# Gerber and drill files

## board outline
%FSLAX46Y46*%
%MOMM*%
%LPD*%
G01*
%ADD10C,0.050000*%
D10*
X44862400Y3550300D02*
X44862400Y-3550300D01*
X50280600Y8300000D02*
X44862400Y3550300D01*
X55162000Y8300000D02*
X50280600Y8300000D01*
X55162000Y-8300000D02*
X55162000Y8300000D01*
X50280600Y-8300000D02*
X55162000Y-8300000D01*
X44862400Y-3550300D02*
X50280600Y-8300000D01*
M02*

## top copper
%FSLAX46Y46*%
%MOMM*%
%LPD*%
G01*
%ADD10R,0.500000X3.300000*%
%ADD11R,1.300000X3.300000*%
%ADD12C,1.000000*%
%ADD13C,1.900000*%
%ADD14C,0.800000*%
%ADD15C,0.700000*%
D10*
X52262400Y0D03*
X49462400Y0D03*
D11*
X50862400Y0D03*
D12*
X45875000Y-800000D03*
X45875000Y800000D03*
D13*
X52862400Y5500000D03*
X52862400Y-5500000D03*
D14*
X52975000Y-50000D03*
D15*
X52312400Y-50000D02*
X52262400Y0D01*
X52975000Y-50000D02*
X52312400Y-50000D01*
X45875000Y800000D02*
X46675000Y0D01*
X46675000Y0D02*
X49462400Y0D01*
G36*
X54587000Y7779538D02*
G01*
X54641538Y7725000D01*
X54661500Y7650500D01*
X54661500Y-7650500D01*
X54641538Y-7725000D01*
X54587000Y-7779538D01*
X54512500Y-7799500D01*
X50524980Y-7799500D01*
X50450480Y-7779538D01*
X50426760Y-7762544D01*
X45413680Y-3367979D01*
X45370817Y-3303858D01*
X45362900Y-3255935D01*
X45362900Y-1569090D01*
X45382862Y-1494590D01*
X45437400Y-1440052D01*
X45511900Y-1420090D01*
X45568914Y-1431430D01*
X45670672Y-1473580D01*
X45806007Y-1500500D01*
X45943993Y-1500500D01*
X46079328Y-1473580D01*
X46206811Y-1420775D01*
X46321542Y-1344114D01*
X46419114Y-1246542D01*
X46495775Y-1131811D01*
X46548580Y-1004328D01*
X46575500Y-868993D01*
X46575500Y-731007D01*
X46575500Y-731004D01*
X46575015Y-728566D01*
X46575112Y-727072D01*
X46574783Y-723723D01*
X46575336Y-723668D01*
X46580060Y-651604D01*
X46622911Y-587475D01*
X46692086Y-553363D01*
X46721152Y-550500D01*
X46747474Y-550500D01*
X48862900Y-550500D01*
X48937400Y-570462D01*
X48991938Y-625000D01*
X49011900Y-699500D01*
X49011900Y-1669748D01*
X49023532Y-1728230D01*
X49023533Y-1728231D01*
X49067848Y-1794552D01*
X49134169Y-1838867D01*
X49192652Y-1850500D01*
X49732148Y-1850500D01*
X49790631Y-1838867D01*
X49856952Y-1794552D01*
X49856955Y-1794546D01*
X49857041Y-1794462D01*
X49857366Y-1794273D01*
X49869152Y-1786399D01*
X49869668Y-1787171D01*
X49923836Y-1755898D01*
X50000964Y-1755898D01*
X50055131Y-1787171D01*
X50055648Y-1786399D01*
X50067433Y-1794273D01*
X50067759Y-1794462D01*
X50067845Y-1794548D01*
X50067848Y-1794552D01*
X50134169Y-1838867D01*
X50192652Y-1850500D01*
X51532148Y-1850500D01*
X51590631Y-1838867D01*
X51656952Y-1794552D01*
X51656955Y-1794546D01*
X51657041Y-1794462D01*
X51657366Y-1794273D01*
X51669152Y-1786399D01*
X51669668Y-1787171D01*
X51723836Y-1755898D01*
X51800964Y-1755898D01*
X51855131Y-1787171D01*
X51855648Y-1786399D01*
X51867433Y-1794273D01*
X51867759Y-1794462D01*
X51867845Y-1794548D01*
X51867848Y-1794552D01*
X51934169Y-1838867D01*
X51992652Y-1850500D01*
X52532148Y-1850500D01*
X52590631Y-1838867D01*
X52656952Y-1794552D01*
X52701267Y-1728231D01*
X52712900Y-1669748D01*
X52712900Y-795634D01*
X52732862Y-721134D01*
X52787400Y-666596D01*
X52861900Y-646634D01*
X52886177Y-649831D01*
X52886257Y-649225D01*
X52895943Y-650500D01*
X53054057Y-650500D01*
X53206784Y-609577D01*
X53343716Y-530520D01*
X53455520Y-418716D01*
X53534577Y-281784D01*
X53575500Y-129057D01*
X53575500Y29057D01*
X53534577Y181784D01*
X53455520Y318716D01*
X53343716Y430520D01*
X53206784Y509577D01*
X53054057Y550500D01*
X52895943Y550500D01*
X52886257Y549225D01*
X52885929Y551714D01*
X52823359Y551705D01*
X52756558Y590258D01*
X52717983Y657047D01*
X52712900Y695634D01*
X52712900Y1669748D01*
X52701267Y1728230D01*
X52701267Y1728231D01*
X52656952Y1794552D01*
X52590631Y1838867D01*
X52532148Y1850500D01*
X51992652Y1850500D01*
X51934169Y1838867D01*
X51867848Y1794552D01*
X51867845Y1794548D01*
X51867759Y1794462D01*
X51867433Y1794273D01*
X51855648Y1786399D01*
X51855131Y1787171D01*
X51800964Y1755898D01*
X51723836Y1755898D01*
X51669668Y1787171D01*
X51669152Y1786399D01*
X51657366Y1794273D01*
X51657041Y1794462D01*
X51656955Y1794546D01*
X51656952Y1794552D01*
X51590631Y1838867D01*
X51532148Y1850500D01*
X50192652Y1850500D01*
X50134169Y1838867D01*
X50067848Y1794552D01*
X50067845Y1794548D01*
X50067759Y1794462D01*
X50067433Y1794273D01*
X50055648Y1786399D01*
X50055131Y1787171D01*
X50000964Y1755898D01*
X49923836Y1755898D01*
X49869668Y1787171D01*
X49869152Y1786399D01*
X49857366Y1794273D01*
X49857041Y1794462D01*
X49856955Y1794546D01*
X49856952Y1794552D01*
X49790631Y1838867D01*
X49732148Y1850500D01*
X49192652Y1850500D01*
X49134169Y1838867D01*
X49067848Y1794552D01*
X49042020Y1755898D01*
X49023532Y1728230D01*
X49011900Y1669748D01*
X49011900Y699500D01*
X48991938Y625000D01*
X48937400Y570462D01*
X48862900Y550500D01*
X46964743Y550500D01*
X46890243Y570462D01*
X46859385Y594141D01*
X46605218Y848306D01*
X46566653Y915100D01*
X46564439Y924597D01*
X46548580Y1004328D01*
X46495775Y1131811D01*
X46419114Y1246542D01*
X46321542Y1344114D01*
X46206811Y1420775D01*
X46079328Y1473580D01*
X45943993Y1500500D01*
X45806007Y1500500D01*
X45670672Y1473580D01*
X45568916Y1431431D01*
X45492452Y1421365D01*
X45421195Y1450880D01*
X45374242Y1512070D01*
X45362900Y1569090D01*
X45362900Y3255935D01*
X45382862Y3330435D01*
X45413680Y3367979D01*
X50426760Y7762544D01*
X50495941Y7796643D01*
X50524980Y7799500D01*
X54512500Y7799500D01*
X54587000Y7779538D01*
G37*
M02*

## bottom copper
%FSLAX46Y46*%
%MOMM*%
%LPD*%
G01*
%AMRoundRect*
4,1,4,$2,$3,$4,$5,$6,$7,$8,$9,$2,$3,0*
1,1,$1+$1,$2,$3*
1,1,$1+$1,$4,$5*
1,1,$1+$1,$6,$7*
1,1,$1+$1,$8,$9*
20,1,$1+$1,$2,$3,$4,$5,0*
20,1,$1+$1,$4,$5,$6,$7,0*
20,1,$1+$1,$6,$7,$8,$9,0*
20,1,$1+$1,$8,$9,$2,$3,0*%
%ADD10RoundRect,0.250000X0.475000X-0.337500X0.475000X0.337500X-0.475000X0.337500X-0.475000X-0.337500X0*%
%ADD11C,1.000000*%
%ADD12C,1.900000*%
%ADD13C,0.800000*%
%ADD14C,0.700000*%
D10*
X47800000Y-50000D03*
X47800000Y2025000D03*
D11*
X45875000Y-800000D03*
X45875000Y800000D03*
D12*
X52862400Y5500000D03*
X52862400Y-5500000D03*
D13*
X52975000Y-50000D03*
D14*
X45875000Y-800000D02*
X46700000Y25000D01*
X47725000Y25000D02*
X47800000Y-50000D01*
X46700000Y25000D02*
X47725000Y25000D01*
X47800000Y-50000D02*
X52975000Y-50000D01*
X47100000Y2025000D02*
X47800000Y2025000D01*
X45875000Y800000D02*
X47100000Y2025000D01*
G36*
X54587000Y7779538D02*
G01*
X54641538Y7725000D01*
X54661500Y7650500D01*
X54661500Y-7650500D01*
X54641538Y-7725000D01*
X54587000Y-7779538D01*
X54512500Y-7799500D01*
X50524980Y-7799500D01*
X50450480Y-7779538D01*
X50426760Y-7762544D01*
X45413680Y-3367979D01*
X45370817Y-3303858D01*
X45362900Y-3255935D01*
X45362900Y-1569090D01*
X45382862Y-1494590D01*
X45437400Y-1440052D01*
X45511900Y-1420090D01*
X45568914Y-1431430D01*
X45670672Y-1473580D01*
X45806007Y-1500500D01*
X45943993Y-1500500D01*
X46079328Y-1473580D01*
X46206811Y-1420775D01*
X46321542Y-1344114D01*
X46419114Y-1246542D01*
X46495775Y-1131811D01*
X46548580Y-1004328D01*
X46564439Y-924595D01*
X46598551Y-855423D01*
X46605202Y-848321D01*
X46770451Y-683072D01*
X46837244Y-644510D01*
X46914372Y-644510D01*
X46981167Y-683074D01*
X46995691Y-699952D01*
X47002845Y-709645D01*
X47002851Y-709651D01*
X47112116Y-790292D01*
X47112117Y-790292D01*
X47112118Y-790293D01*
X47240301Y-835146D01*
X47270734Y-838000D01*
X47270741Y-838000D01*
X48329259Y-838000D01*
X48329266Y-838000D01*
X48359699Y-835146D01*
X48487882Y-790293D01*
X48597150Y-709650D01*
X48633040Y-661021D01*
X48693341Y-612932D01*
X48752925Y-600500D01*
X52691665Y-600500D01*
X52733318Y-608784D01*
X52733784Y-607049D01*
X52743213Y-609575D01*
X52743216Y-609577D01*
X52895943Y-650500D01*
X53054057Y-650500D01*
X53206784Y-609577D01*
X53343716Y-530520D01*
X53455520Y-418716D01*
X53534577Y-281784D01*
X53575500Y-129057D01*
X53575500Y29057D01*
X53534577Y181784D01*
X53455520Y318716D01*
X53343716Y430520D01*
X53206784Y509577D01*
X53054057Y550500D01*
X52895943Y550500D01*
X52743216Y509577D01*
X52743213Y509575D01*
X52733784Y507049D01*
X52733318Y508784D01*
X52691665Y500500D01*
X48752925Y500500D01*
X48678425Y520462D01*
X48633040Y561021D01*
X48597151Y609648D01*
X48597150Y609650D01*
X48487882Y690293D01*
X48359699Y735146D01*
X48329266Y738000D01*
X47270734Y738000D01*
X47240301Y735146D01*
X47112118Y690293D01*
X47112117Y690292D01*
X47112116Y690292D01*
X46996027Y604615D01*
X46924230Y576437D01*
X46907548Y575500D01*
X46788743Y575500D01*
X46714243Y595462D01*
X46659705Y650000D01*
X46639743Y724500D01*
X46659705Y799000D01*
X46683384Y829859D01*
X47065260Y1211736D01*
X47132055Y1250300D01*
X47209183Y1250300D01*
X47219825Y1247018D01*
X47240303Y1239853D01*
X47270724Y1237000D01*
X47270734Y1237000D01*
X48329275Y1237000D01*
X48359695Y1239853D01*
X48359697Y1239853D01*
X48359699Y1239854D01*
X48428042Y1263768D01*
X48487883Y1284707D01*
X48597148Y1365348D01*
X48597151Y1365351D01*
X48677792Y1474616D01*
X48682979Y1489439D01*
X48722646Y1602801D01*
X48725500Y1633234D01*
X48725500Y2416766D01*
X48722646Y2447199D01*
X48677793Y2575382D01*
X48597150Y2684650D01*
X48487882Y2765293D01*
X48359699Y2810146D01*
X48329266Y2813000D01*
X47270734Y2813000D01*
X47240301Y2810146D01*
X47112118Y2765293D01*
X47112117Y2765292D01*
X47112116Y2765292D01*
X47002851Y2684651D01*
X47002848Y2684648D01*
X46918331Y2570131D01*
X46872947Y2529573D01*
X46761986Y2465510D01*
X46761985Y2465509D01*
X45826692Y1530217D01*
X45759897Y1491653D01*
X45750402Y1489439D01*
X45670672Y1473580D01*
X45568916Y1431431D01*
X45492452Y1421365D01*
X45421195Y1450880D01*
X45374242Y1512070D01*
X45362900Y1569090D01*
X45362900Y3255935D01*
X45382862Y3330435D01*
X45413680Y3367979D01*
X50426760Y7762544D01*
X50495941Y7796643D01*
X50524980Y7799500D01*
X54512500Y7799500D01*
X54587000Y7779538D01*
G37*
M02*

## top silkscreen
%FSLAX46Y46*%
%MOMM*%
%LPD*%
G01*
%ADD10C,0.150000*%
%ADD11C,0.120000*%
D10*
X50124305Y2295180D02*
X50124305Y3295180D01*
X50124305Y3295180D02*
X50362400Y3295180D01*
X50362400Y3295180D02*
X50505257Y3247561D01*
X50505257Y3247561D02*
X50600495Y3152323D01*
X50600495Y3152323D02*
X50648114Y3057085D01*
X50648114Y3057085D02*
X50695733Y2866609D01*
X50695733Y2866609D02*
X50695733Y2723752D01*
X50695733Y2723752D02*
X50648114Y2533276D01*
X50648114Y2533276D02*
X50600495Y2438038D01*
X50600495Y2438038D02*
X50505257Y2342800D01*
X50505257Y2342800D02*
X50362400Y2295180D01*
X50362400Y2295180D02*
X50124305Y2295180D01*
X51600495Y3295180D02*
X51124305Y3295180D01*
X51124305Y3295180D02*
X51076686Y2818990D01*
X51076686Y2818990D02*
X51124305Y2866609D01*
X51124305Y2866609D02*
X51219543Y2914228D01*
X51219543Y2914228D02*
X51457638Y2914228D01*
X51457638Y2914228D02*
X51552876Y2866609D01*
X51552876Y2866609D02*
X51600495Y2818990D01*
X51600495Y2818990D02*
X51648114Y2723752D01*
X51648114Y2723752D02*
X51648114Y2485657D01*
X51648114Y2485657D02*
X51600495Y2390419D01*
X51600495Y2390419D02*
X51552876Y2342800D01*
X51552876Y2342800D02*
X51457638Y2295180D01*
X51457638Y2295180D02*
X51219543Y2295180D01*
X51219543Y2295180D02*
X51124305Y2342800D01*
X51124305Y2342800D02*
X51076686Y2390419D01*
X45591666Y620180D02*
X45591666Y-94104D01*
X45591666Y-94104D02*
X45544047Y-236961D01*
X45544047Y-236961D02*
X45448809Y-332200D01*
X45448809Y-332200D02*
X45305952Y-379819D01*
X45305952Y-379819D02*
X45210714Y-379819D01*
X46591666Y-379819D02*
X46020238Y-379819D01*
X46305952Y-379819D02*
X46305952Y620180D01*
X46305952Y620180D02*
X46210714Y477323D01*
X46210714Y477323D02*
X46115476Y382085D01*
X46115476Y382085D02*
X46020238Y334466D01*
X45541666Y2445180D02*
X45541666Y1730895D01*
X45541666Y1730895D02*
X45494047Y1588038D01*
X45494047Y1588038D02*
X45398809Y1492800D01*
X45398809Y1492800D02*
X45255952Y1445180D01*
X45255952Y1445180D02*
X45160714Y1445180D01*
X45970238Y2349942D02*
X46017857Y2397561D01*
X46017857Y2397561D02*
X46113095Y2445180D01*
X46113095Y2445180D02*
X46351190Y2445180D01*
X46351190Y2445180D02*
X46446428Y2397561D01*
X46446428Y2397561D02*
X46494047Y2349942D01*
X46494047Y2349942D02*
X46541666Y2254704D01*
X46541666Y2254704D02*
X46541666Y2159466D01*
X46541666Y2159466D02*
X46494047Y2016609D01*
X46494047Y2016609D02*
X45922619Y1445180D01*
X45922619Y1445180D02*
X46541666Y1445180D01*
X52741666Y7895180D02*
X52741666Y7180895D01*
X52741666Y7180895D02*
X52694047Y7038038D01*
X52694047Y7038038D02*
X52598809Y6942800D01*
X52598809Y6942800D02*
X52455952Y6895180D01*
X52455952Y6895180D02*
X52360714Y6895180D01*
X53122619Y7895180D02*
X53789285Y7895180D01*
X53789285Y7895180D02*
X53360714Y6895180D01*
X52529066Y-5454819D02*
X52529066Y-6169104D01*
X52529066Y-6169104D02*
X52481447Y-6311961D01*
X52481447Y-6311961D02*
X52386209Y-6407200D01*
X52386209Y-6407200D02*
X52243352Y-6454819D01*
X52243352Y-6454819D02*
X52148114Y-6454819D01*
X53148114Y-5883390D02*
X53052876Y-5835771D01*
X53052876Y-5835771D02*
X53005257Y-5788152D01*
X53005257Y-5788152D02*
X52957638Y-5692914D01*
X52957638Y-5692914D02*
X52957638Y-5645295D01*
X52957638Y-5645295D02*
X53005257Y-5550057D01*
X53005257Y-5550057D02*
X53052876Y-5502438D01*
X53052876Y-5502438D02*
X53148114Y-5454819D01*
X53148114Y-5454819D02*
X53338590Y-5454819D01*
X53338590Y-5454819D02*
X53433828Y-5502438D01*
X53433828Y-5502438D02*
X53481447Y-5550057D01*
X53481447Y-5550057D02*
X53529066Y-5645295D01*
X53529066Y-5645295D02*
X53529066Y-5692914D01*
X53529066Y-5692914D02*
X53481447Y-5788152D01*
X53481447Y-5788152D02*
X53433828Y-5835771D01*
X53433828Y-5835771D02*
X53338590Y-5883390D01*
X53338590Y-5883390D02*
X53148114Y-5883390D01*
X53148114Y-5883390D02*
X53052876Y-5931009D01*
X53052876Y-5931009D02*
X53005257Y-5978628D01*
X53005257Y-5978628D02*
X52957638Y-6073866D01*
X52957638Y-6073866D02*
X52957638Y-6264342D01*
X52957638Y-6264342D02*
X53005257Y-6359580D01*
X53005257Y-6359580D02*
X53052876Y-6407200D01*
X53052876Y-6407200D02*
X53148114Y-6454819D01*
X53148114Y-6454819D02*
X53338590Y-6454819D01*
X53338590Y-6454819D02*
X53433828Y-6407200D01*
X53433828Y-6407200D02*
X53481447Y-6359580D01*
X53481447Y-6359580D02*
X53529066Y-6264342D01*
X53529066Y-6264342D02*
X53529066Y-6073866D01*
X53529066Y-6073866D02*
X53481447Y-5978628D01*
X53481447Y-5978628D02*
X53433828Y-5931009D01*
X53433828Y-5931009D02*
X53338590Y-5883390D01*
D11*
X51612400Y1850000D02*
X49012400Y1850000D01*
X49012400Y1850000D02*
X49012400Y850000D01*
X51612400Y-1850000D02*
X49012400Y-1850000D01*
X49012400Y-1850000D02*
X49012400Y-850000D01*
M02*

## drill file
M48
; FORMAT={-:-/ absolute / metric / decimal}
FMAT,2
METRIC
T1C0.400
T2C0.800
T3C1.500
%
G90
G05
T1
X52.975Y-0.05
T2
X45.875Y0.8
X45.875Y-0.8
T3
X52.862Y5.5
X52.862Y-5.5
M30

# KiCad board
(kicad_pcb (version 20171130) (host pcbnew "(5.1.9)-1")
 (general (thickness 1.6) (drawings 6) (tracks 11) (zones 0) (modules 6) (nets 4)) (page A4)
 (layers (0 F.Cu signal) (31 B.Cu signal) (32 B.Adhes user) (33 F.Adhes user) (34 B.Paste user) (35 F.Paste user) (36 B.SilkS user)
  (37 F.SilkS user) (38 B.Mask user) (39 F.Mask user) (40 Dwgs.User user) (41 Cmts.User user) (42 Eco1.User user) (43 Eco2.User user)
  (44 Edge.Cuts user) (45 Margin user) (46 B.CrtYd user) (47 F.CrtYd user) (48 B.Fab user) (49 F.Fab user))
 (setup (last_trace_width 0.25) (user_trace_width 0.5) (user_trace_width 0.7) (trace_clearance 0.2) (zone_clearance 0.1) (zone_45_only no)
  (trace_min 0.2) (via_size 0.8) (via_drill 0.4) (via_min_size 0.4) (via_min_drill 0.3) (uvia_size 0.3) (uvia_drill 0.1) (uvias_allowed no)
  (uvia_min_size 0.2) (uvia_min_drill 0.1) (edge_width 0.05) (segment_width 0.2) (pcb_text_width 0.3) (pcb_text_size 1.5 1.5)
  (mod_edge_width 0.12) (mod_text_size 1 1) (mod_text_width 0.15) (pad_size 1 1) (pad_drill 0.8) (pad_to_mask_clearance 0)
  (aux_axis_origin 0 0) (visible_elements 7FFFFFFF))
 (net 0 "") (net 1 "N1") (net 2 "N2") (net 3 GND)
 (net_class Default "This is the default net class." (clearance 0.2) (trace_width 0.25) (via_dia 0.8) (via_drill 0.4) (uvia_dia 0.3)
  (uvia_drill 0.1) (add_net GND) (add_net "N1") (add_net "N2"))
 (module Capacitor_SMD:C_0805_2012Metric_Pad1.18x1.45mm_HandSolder (layer B.Cu) (at 47.8 -0.9875 90)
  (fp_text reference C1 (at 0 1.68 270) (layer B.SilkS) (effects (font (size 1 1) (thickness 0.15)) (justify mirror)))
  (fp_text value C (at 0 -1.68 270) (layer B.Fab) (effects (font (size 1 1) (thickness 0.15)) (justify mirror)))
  (pad 1 smd roundrect (at -1.0375 0 90) (size 1.175 1.45) (layers B.Cu B.Paste B.Mask) (roundrect_rratio 0.2127659574468085) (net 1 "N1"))
  (pad 2 smd roundrect (at 1.0375 0 90) (size 1.175 1.45) (layers B.Cu B.Paste B.Mask) (roundrect_rratio 0.2127659574468085) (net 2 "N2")))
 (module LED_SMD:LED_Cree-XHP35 (layer F.Cu) (at 50.8624 0)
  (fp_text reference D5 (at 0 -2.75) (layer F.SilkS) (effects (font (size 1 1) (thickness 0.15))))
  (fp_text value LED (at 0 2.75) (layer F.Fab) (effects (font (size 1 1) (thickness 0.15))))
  (fp_line (start 0.75 -1.85) (end -1.85 -1.85) (layer F.SilkS) (width 0.12))
  (fp_line (start -1.85 -1.85) (end -1.85 -0.85) (layer F.SilkS) (width 0.12))
  (fp_line (start 0.75 1.85) (end -1.85 1.85) (layer F.SilkS) (width 0.12))
  (fp_line (start -1.85 1.85) (end -1.85 0.85) (layer F.SilkS) (width 0.12))
  (pad 2 smd rect (at 1.4 0) (size 0.5 3.3) (layers F.Cu F.Paste F.Mask) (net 1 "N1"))
  (pad 1 smd rect (at -1.4 0) (size 0.5 3.3) (layers F.Cu F.Paste F.Mask) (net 2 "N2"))
  (pad 3 smd rect (at 0 0) (size 1.3 3.3) (layers F.Cu F.Mask)) (pad "" smd rect (at 0 1) (size 1.01 0.75) (layers F.Paste))
  (pad "" smd rect (at 0 -1) (size 1.01 0.75) (layers F.Paste)) (pad "" smd rect (at 0 0) (size 1.01 0.75) (layers F.Paste)))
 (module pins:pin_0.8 (layer F.Cu) (at 45.925 -0.575)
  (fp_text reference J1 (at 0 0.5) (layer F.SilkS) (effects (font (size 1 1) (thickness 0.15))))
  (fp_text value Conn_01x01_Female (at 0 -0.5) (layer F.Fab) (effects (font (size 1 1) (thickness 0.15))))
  (pad 1 thru_hole circle (at -0.05 1.375) (size 1 1) (drill 0.8) (layers *.Cu *.Mask) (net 1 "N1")))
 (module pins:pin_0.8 (layer F.Cu) (at 45.875 -2.4)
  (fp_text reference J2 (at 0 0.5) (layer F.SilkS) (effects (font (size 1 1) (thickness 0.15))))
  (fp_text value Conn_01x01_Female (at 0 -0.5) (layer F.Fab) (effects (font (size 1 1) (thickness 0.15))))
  (pad 1 thru_hole circle (at 0 1.6) (size 1 1) (drill 0.8) (layers *.Cu *.Mask) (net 2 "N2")))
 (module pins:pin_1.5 (layer F.Cu) (at 53.075 -7.85)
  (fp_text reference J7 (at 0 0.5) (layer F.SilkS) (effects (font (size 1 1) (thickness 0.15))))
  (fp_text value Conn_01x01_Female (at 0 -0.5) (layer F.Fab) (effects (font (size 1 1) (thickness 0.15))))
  (pad 1 thru_hole circle (at -0.2126 2.35) (size 1.9 1.9) (drill 1.5) (layers *.Cu *.Mask) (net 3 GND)))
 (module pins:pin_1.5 (layer F.Cu) (at 52.8624 5.5)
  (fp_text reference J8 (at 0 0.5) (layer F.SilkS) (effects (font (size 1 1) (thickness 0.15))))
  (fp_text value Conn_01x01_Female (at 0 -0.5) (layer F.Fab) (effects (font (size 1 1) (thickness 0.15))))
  (pad 1 thru_hole circle (at 0 0) (size 1.9 1.9) (drill 1.5) (layers *.Cu *.Mask) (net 3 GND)))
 (gr_line (start 44.8624 -3.5503) (end 44.8624 3.5503) (layer Edge.Cuts) (width 0.05))
 (gr_line (start 50.2806 -8.3) (end 44.8624 -3.5503) (layer Edge.Cuts) (width 0.05))
 (gr_line (start 55.162 -8.3) (end 50.2806 -8.3) (layer Edge.Cuts) (width 0.05))
 (gr_line (start 55.162 8.3) (end 55.162 -8.3) (layer Edge.Cuts) (width 0.05))
 (gr_line (start 50.2806 8.3) (end 55.162 8.3) (layer Edge.Cuts) (width 0.05))
 (gr_line (start 44.8624 3.5503) (end 50.2806 8.3) (layer Edge.Cuts) (width 0.05))
 (segment (start 45.875 0.8) (end 46.7 -0.025) (width 0.7) (layer B.Cu) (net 1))
 (segment (start 47.725 -0.025) (end 47.8 0.05) (width 0.7) (layer B.Cu) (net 1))
 (segment (start 46.7 -0.025) (end 47.725 -0.025) (width 0.7) (layer B.Cu) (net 1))
 (segment (start 47.8 0.05) (end 52.975 0.05) (width 0.7) (layer B.Cu) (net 1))
 (via (at 52.975 0.05) (size 0.8) (drill 0.4) (layers F.Cu B.Cu) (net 1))
 (segment (start 52.3124 0.05) (end 52.2624 0) (width 0.7) (layer F.Cu) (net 1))
 (segment (start 52.975 0.05) (end 52.3124 0.05) (width 0.7) (layer F.Cu) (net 1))
 (segment (start 45.875 -0.8) (end 46.675 0) (width 0.7) (layer F.Cu) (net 2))
 (segment (start 46.675 0) (end 49.4624 0) (width 0.7) (layer F.Cu) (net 2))
 (segment (start 47.1 -2.025) (end 47.8 -2.025) (width 0.7) (layer B.Cu) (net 2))
 (segment (start 45.875 -0.8) (end 47.1 -2.025) (width 0.7) (layer B.Cu) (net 2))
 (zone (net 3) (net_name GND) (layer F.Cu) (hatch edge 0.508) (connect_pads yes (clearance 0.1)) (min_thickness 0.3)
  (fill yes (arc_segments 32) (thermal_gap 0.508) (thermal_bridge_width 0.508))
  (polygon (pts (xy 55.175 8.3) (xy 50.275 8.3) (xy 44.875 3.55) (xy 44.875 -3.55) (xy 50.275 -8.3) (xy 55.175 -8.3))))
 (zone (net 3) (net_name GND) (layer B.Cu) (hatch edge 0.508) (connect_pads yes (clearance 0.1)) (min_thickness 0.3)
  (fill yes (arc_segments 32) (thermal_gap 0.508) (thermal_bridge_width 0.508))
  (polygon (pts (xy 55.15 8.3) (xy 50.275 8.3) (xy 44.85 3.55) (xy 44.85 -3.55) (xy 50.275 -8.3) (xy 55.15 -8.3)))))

